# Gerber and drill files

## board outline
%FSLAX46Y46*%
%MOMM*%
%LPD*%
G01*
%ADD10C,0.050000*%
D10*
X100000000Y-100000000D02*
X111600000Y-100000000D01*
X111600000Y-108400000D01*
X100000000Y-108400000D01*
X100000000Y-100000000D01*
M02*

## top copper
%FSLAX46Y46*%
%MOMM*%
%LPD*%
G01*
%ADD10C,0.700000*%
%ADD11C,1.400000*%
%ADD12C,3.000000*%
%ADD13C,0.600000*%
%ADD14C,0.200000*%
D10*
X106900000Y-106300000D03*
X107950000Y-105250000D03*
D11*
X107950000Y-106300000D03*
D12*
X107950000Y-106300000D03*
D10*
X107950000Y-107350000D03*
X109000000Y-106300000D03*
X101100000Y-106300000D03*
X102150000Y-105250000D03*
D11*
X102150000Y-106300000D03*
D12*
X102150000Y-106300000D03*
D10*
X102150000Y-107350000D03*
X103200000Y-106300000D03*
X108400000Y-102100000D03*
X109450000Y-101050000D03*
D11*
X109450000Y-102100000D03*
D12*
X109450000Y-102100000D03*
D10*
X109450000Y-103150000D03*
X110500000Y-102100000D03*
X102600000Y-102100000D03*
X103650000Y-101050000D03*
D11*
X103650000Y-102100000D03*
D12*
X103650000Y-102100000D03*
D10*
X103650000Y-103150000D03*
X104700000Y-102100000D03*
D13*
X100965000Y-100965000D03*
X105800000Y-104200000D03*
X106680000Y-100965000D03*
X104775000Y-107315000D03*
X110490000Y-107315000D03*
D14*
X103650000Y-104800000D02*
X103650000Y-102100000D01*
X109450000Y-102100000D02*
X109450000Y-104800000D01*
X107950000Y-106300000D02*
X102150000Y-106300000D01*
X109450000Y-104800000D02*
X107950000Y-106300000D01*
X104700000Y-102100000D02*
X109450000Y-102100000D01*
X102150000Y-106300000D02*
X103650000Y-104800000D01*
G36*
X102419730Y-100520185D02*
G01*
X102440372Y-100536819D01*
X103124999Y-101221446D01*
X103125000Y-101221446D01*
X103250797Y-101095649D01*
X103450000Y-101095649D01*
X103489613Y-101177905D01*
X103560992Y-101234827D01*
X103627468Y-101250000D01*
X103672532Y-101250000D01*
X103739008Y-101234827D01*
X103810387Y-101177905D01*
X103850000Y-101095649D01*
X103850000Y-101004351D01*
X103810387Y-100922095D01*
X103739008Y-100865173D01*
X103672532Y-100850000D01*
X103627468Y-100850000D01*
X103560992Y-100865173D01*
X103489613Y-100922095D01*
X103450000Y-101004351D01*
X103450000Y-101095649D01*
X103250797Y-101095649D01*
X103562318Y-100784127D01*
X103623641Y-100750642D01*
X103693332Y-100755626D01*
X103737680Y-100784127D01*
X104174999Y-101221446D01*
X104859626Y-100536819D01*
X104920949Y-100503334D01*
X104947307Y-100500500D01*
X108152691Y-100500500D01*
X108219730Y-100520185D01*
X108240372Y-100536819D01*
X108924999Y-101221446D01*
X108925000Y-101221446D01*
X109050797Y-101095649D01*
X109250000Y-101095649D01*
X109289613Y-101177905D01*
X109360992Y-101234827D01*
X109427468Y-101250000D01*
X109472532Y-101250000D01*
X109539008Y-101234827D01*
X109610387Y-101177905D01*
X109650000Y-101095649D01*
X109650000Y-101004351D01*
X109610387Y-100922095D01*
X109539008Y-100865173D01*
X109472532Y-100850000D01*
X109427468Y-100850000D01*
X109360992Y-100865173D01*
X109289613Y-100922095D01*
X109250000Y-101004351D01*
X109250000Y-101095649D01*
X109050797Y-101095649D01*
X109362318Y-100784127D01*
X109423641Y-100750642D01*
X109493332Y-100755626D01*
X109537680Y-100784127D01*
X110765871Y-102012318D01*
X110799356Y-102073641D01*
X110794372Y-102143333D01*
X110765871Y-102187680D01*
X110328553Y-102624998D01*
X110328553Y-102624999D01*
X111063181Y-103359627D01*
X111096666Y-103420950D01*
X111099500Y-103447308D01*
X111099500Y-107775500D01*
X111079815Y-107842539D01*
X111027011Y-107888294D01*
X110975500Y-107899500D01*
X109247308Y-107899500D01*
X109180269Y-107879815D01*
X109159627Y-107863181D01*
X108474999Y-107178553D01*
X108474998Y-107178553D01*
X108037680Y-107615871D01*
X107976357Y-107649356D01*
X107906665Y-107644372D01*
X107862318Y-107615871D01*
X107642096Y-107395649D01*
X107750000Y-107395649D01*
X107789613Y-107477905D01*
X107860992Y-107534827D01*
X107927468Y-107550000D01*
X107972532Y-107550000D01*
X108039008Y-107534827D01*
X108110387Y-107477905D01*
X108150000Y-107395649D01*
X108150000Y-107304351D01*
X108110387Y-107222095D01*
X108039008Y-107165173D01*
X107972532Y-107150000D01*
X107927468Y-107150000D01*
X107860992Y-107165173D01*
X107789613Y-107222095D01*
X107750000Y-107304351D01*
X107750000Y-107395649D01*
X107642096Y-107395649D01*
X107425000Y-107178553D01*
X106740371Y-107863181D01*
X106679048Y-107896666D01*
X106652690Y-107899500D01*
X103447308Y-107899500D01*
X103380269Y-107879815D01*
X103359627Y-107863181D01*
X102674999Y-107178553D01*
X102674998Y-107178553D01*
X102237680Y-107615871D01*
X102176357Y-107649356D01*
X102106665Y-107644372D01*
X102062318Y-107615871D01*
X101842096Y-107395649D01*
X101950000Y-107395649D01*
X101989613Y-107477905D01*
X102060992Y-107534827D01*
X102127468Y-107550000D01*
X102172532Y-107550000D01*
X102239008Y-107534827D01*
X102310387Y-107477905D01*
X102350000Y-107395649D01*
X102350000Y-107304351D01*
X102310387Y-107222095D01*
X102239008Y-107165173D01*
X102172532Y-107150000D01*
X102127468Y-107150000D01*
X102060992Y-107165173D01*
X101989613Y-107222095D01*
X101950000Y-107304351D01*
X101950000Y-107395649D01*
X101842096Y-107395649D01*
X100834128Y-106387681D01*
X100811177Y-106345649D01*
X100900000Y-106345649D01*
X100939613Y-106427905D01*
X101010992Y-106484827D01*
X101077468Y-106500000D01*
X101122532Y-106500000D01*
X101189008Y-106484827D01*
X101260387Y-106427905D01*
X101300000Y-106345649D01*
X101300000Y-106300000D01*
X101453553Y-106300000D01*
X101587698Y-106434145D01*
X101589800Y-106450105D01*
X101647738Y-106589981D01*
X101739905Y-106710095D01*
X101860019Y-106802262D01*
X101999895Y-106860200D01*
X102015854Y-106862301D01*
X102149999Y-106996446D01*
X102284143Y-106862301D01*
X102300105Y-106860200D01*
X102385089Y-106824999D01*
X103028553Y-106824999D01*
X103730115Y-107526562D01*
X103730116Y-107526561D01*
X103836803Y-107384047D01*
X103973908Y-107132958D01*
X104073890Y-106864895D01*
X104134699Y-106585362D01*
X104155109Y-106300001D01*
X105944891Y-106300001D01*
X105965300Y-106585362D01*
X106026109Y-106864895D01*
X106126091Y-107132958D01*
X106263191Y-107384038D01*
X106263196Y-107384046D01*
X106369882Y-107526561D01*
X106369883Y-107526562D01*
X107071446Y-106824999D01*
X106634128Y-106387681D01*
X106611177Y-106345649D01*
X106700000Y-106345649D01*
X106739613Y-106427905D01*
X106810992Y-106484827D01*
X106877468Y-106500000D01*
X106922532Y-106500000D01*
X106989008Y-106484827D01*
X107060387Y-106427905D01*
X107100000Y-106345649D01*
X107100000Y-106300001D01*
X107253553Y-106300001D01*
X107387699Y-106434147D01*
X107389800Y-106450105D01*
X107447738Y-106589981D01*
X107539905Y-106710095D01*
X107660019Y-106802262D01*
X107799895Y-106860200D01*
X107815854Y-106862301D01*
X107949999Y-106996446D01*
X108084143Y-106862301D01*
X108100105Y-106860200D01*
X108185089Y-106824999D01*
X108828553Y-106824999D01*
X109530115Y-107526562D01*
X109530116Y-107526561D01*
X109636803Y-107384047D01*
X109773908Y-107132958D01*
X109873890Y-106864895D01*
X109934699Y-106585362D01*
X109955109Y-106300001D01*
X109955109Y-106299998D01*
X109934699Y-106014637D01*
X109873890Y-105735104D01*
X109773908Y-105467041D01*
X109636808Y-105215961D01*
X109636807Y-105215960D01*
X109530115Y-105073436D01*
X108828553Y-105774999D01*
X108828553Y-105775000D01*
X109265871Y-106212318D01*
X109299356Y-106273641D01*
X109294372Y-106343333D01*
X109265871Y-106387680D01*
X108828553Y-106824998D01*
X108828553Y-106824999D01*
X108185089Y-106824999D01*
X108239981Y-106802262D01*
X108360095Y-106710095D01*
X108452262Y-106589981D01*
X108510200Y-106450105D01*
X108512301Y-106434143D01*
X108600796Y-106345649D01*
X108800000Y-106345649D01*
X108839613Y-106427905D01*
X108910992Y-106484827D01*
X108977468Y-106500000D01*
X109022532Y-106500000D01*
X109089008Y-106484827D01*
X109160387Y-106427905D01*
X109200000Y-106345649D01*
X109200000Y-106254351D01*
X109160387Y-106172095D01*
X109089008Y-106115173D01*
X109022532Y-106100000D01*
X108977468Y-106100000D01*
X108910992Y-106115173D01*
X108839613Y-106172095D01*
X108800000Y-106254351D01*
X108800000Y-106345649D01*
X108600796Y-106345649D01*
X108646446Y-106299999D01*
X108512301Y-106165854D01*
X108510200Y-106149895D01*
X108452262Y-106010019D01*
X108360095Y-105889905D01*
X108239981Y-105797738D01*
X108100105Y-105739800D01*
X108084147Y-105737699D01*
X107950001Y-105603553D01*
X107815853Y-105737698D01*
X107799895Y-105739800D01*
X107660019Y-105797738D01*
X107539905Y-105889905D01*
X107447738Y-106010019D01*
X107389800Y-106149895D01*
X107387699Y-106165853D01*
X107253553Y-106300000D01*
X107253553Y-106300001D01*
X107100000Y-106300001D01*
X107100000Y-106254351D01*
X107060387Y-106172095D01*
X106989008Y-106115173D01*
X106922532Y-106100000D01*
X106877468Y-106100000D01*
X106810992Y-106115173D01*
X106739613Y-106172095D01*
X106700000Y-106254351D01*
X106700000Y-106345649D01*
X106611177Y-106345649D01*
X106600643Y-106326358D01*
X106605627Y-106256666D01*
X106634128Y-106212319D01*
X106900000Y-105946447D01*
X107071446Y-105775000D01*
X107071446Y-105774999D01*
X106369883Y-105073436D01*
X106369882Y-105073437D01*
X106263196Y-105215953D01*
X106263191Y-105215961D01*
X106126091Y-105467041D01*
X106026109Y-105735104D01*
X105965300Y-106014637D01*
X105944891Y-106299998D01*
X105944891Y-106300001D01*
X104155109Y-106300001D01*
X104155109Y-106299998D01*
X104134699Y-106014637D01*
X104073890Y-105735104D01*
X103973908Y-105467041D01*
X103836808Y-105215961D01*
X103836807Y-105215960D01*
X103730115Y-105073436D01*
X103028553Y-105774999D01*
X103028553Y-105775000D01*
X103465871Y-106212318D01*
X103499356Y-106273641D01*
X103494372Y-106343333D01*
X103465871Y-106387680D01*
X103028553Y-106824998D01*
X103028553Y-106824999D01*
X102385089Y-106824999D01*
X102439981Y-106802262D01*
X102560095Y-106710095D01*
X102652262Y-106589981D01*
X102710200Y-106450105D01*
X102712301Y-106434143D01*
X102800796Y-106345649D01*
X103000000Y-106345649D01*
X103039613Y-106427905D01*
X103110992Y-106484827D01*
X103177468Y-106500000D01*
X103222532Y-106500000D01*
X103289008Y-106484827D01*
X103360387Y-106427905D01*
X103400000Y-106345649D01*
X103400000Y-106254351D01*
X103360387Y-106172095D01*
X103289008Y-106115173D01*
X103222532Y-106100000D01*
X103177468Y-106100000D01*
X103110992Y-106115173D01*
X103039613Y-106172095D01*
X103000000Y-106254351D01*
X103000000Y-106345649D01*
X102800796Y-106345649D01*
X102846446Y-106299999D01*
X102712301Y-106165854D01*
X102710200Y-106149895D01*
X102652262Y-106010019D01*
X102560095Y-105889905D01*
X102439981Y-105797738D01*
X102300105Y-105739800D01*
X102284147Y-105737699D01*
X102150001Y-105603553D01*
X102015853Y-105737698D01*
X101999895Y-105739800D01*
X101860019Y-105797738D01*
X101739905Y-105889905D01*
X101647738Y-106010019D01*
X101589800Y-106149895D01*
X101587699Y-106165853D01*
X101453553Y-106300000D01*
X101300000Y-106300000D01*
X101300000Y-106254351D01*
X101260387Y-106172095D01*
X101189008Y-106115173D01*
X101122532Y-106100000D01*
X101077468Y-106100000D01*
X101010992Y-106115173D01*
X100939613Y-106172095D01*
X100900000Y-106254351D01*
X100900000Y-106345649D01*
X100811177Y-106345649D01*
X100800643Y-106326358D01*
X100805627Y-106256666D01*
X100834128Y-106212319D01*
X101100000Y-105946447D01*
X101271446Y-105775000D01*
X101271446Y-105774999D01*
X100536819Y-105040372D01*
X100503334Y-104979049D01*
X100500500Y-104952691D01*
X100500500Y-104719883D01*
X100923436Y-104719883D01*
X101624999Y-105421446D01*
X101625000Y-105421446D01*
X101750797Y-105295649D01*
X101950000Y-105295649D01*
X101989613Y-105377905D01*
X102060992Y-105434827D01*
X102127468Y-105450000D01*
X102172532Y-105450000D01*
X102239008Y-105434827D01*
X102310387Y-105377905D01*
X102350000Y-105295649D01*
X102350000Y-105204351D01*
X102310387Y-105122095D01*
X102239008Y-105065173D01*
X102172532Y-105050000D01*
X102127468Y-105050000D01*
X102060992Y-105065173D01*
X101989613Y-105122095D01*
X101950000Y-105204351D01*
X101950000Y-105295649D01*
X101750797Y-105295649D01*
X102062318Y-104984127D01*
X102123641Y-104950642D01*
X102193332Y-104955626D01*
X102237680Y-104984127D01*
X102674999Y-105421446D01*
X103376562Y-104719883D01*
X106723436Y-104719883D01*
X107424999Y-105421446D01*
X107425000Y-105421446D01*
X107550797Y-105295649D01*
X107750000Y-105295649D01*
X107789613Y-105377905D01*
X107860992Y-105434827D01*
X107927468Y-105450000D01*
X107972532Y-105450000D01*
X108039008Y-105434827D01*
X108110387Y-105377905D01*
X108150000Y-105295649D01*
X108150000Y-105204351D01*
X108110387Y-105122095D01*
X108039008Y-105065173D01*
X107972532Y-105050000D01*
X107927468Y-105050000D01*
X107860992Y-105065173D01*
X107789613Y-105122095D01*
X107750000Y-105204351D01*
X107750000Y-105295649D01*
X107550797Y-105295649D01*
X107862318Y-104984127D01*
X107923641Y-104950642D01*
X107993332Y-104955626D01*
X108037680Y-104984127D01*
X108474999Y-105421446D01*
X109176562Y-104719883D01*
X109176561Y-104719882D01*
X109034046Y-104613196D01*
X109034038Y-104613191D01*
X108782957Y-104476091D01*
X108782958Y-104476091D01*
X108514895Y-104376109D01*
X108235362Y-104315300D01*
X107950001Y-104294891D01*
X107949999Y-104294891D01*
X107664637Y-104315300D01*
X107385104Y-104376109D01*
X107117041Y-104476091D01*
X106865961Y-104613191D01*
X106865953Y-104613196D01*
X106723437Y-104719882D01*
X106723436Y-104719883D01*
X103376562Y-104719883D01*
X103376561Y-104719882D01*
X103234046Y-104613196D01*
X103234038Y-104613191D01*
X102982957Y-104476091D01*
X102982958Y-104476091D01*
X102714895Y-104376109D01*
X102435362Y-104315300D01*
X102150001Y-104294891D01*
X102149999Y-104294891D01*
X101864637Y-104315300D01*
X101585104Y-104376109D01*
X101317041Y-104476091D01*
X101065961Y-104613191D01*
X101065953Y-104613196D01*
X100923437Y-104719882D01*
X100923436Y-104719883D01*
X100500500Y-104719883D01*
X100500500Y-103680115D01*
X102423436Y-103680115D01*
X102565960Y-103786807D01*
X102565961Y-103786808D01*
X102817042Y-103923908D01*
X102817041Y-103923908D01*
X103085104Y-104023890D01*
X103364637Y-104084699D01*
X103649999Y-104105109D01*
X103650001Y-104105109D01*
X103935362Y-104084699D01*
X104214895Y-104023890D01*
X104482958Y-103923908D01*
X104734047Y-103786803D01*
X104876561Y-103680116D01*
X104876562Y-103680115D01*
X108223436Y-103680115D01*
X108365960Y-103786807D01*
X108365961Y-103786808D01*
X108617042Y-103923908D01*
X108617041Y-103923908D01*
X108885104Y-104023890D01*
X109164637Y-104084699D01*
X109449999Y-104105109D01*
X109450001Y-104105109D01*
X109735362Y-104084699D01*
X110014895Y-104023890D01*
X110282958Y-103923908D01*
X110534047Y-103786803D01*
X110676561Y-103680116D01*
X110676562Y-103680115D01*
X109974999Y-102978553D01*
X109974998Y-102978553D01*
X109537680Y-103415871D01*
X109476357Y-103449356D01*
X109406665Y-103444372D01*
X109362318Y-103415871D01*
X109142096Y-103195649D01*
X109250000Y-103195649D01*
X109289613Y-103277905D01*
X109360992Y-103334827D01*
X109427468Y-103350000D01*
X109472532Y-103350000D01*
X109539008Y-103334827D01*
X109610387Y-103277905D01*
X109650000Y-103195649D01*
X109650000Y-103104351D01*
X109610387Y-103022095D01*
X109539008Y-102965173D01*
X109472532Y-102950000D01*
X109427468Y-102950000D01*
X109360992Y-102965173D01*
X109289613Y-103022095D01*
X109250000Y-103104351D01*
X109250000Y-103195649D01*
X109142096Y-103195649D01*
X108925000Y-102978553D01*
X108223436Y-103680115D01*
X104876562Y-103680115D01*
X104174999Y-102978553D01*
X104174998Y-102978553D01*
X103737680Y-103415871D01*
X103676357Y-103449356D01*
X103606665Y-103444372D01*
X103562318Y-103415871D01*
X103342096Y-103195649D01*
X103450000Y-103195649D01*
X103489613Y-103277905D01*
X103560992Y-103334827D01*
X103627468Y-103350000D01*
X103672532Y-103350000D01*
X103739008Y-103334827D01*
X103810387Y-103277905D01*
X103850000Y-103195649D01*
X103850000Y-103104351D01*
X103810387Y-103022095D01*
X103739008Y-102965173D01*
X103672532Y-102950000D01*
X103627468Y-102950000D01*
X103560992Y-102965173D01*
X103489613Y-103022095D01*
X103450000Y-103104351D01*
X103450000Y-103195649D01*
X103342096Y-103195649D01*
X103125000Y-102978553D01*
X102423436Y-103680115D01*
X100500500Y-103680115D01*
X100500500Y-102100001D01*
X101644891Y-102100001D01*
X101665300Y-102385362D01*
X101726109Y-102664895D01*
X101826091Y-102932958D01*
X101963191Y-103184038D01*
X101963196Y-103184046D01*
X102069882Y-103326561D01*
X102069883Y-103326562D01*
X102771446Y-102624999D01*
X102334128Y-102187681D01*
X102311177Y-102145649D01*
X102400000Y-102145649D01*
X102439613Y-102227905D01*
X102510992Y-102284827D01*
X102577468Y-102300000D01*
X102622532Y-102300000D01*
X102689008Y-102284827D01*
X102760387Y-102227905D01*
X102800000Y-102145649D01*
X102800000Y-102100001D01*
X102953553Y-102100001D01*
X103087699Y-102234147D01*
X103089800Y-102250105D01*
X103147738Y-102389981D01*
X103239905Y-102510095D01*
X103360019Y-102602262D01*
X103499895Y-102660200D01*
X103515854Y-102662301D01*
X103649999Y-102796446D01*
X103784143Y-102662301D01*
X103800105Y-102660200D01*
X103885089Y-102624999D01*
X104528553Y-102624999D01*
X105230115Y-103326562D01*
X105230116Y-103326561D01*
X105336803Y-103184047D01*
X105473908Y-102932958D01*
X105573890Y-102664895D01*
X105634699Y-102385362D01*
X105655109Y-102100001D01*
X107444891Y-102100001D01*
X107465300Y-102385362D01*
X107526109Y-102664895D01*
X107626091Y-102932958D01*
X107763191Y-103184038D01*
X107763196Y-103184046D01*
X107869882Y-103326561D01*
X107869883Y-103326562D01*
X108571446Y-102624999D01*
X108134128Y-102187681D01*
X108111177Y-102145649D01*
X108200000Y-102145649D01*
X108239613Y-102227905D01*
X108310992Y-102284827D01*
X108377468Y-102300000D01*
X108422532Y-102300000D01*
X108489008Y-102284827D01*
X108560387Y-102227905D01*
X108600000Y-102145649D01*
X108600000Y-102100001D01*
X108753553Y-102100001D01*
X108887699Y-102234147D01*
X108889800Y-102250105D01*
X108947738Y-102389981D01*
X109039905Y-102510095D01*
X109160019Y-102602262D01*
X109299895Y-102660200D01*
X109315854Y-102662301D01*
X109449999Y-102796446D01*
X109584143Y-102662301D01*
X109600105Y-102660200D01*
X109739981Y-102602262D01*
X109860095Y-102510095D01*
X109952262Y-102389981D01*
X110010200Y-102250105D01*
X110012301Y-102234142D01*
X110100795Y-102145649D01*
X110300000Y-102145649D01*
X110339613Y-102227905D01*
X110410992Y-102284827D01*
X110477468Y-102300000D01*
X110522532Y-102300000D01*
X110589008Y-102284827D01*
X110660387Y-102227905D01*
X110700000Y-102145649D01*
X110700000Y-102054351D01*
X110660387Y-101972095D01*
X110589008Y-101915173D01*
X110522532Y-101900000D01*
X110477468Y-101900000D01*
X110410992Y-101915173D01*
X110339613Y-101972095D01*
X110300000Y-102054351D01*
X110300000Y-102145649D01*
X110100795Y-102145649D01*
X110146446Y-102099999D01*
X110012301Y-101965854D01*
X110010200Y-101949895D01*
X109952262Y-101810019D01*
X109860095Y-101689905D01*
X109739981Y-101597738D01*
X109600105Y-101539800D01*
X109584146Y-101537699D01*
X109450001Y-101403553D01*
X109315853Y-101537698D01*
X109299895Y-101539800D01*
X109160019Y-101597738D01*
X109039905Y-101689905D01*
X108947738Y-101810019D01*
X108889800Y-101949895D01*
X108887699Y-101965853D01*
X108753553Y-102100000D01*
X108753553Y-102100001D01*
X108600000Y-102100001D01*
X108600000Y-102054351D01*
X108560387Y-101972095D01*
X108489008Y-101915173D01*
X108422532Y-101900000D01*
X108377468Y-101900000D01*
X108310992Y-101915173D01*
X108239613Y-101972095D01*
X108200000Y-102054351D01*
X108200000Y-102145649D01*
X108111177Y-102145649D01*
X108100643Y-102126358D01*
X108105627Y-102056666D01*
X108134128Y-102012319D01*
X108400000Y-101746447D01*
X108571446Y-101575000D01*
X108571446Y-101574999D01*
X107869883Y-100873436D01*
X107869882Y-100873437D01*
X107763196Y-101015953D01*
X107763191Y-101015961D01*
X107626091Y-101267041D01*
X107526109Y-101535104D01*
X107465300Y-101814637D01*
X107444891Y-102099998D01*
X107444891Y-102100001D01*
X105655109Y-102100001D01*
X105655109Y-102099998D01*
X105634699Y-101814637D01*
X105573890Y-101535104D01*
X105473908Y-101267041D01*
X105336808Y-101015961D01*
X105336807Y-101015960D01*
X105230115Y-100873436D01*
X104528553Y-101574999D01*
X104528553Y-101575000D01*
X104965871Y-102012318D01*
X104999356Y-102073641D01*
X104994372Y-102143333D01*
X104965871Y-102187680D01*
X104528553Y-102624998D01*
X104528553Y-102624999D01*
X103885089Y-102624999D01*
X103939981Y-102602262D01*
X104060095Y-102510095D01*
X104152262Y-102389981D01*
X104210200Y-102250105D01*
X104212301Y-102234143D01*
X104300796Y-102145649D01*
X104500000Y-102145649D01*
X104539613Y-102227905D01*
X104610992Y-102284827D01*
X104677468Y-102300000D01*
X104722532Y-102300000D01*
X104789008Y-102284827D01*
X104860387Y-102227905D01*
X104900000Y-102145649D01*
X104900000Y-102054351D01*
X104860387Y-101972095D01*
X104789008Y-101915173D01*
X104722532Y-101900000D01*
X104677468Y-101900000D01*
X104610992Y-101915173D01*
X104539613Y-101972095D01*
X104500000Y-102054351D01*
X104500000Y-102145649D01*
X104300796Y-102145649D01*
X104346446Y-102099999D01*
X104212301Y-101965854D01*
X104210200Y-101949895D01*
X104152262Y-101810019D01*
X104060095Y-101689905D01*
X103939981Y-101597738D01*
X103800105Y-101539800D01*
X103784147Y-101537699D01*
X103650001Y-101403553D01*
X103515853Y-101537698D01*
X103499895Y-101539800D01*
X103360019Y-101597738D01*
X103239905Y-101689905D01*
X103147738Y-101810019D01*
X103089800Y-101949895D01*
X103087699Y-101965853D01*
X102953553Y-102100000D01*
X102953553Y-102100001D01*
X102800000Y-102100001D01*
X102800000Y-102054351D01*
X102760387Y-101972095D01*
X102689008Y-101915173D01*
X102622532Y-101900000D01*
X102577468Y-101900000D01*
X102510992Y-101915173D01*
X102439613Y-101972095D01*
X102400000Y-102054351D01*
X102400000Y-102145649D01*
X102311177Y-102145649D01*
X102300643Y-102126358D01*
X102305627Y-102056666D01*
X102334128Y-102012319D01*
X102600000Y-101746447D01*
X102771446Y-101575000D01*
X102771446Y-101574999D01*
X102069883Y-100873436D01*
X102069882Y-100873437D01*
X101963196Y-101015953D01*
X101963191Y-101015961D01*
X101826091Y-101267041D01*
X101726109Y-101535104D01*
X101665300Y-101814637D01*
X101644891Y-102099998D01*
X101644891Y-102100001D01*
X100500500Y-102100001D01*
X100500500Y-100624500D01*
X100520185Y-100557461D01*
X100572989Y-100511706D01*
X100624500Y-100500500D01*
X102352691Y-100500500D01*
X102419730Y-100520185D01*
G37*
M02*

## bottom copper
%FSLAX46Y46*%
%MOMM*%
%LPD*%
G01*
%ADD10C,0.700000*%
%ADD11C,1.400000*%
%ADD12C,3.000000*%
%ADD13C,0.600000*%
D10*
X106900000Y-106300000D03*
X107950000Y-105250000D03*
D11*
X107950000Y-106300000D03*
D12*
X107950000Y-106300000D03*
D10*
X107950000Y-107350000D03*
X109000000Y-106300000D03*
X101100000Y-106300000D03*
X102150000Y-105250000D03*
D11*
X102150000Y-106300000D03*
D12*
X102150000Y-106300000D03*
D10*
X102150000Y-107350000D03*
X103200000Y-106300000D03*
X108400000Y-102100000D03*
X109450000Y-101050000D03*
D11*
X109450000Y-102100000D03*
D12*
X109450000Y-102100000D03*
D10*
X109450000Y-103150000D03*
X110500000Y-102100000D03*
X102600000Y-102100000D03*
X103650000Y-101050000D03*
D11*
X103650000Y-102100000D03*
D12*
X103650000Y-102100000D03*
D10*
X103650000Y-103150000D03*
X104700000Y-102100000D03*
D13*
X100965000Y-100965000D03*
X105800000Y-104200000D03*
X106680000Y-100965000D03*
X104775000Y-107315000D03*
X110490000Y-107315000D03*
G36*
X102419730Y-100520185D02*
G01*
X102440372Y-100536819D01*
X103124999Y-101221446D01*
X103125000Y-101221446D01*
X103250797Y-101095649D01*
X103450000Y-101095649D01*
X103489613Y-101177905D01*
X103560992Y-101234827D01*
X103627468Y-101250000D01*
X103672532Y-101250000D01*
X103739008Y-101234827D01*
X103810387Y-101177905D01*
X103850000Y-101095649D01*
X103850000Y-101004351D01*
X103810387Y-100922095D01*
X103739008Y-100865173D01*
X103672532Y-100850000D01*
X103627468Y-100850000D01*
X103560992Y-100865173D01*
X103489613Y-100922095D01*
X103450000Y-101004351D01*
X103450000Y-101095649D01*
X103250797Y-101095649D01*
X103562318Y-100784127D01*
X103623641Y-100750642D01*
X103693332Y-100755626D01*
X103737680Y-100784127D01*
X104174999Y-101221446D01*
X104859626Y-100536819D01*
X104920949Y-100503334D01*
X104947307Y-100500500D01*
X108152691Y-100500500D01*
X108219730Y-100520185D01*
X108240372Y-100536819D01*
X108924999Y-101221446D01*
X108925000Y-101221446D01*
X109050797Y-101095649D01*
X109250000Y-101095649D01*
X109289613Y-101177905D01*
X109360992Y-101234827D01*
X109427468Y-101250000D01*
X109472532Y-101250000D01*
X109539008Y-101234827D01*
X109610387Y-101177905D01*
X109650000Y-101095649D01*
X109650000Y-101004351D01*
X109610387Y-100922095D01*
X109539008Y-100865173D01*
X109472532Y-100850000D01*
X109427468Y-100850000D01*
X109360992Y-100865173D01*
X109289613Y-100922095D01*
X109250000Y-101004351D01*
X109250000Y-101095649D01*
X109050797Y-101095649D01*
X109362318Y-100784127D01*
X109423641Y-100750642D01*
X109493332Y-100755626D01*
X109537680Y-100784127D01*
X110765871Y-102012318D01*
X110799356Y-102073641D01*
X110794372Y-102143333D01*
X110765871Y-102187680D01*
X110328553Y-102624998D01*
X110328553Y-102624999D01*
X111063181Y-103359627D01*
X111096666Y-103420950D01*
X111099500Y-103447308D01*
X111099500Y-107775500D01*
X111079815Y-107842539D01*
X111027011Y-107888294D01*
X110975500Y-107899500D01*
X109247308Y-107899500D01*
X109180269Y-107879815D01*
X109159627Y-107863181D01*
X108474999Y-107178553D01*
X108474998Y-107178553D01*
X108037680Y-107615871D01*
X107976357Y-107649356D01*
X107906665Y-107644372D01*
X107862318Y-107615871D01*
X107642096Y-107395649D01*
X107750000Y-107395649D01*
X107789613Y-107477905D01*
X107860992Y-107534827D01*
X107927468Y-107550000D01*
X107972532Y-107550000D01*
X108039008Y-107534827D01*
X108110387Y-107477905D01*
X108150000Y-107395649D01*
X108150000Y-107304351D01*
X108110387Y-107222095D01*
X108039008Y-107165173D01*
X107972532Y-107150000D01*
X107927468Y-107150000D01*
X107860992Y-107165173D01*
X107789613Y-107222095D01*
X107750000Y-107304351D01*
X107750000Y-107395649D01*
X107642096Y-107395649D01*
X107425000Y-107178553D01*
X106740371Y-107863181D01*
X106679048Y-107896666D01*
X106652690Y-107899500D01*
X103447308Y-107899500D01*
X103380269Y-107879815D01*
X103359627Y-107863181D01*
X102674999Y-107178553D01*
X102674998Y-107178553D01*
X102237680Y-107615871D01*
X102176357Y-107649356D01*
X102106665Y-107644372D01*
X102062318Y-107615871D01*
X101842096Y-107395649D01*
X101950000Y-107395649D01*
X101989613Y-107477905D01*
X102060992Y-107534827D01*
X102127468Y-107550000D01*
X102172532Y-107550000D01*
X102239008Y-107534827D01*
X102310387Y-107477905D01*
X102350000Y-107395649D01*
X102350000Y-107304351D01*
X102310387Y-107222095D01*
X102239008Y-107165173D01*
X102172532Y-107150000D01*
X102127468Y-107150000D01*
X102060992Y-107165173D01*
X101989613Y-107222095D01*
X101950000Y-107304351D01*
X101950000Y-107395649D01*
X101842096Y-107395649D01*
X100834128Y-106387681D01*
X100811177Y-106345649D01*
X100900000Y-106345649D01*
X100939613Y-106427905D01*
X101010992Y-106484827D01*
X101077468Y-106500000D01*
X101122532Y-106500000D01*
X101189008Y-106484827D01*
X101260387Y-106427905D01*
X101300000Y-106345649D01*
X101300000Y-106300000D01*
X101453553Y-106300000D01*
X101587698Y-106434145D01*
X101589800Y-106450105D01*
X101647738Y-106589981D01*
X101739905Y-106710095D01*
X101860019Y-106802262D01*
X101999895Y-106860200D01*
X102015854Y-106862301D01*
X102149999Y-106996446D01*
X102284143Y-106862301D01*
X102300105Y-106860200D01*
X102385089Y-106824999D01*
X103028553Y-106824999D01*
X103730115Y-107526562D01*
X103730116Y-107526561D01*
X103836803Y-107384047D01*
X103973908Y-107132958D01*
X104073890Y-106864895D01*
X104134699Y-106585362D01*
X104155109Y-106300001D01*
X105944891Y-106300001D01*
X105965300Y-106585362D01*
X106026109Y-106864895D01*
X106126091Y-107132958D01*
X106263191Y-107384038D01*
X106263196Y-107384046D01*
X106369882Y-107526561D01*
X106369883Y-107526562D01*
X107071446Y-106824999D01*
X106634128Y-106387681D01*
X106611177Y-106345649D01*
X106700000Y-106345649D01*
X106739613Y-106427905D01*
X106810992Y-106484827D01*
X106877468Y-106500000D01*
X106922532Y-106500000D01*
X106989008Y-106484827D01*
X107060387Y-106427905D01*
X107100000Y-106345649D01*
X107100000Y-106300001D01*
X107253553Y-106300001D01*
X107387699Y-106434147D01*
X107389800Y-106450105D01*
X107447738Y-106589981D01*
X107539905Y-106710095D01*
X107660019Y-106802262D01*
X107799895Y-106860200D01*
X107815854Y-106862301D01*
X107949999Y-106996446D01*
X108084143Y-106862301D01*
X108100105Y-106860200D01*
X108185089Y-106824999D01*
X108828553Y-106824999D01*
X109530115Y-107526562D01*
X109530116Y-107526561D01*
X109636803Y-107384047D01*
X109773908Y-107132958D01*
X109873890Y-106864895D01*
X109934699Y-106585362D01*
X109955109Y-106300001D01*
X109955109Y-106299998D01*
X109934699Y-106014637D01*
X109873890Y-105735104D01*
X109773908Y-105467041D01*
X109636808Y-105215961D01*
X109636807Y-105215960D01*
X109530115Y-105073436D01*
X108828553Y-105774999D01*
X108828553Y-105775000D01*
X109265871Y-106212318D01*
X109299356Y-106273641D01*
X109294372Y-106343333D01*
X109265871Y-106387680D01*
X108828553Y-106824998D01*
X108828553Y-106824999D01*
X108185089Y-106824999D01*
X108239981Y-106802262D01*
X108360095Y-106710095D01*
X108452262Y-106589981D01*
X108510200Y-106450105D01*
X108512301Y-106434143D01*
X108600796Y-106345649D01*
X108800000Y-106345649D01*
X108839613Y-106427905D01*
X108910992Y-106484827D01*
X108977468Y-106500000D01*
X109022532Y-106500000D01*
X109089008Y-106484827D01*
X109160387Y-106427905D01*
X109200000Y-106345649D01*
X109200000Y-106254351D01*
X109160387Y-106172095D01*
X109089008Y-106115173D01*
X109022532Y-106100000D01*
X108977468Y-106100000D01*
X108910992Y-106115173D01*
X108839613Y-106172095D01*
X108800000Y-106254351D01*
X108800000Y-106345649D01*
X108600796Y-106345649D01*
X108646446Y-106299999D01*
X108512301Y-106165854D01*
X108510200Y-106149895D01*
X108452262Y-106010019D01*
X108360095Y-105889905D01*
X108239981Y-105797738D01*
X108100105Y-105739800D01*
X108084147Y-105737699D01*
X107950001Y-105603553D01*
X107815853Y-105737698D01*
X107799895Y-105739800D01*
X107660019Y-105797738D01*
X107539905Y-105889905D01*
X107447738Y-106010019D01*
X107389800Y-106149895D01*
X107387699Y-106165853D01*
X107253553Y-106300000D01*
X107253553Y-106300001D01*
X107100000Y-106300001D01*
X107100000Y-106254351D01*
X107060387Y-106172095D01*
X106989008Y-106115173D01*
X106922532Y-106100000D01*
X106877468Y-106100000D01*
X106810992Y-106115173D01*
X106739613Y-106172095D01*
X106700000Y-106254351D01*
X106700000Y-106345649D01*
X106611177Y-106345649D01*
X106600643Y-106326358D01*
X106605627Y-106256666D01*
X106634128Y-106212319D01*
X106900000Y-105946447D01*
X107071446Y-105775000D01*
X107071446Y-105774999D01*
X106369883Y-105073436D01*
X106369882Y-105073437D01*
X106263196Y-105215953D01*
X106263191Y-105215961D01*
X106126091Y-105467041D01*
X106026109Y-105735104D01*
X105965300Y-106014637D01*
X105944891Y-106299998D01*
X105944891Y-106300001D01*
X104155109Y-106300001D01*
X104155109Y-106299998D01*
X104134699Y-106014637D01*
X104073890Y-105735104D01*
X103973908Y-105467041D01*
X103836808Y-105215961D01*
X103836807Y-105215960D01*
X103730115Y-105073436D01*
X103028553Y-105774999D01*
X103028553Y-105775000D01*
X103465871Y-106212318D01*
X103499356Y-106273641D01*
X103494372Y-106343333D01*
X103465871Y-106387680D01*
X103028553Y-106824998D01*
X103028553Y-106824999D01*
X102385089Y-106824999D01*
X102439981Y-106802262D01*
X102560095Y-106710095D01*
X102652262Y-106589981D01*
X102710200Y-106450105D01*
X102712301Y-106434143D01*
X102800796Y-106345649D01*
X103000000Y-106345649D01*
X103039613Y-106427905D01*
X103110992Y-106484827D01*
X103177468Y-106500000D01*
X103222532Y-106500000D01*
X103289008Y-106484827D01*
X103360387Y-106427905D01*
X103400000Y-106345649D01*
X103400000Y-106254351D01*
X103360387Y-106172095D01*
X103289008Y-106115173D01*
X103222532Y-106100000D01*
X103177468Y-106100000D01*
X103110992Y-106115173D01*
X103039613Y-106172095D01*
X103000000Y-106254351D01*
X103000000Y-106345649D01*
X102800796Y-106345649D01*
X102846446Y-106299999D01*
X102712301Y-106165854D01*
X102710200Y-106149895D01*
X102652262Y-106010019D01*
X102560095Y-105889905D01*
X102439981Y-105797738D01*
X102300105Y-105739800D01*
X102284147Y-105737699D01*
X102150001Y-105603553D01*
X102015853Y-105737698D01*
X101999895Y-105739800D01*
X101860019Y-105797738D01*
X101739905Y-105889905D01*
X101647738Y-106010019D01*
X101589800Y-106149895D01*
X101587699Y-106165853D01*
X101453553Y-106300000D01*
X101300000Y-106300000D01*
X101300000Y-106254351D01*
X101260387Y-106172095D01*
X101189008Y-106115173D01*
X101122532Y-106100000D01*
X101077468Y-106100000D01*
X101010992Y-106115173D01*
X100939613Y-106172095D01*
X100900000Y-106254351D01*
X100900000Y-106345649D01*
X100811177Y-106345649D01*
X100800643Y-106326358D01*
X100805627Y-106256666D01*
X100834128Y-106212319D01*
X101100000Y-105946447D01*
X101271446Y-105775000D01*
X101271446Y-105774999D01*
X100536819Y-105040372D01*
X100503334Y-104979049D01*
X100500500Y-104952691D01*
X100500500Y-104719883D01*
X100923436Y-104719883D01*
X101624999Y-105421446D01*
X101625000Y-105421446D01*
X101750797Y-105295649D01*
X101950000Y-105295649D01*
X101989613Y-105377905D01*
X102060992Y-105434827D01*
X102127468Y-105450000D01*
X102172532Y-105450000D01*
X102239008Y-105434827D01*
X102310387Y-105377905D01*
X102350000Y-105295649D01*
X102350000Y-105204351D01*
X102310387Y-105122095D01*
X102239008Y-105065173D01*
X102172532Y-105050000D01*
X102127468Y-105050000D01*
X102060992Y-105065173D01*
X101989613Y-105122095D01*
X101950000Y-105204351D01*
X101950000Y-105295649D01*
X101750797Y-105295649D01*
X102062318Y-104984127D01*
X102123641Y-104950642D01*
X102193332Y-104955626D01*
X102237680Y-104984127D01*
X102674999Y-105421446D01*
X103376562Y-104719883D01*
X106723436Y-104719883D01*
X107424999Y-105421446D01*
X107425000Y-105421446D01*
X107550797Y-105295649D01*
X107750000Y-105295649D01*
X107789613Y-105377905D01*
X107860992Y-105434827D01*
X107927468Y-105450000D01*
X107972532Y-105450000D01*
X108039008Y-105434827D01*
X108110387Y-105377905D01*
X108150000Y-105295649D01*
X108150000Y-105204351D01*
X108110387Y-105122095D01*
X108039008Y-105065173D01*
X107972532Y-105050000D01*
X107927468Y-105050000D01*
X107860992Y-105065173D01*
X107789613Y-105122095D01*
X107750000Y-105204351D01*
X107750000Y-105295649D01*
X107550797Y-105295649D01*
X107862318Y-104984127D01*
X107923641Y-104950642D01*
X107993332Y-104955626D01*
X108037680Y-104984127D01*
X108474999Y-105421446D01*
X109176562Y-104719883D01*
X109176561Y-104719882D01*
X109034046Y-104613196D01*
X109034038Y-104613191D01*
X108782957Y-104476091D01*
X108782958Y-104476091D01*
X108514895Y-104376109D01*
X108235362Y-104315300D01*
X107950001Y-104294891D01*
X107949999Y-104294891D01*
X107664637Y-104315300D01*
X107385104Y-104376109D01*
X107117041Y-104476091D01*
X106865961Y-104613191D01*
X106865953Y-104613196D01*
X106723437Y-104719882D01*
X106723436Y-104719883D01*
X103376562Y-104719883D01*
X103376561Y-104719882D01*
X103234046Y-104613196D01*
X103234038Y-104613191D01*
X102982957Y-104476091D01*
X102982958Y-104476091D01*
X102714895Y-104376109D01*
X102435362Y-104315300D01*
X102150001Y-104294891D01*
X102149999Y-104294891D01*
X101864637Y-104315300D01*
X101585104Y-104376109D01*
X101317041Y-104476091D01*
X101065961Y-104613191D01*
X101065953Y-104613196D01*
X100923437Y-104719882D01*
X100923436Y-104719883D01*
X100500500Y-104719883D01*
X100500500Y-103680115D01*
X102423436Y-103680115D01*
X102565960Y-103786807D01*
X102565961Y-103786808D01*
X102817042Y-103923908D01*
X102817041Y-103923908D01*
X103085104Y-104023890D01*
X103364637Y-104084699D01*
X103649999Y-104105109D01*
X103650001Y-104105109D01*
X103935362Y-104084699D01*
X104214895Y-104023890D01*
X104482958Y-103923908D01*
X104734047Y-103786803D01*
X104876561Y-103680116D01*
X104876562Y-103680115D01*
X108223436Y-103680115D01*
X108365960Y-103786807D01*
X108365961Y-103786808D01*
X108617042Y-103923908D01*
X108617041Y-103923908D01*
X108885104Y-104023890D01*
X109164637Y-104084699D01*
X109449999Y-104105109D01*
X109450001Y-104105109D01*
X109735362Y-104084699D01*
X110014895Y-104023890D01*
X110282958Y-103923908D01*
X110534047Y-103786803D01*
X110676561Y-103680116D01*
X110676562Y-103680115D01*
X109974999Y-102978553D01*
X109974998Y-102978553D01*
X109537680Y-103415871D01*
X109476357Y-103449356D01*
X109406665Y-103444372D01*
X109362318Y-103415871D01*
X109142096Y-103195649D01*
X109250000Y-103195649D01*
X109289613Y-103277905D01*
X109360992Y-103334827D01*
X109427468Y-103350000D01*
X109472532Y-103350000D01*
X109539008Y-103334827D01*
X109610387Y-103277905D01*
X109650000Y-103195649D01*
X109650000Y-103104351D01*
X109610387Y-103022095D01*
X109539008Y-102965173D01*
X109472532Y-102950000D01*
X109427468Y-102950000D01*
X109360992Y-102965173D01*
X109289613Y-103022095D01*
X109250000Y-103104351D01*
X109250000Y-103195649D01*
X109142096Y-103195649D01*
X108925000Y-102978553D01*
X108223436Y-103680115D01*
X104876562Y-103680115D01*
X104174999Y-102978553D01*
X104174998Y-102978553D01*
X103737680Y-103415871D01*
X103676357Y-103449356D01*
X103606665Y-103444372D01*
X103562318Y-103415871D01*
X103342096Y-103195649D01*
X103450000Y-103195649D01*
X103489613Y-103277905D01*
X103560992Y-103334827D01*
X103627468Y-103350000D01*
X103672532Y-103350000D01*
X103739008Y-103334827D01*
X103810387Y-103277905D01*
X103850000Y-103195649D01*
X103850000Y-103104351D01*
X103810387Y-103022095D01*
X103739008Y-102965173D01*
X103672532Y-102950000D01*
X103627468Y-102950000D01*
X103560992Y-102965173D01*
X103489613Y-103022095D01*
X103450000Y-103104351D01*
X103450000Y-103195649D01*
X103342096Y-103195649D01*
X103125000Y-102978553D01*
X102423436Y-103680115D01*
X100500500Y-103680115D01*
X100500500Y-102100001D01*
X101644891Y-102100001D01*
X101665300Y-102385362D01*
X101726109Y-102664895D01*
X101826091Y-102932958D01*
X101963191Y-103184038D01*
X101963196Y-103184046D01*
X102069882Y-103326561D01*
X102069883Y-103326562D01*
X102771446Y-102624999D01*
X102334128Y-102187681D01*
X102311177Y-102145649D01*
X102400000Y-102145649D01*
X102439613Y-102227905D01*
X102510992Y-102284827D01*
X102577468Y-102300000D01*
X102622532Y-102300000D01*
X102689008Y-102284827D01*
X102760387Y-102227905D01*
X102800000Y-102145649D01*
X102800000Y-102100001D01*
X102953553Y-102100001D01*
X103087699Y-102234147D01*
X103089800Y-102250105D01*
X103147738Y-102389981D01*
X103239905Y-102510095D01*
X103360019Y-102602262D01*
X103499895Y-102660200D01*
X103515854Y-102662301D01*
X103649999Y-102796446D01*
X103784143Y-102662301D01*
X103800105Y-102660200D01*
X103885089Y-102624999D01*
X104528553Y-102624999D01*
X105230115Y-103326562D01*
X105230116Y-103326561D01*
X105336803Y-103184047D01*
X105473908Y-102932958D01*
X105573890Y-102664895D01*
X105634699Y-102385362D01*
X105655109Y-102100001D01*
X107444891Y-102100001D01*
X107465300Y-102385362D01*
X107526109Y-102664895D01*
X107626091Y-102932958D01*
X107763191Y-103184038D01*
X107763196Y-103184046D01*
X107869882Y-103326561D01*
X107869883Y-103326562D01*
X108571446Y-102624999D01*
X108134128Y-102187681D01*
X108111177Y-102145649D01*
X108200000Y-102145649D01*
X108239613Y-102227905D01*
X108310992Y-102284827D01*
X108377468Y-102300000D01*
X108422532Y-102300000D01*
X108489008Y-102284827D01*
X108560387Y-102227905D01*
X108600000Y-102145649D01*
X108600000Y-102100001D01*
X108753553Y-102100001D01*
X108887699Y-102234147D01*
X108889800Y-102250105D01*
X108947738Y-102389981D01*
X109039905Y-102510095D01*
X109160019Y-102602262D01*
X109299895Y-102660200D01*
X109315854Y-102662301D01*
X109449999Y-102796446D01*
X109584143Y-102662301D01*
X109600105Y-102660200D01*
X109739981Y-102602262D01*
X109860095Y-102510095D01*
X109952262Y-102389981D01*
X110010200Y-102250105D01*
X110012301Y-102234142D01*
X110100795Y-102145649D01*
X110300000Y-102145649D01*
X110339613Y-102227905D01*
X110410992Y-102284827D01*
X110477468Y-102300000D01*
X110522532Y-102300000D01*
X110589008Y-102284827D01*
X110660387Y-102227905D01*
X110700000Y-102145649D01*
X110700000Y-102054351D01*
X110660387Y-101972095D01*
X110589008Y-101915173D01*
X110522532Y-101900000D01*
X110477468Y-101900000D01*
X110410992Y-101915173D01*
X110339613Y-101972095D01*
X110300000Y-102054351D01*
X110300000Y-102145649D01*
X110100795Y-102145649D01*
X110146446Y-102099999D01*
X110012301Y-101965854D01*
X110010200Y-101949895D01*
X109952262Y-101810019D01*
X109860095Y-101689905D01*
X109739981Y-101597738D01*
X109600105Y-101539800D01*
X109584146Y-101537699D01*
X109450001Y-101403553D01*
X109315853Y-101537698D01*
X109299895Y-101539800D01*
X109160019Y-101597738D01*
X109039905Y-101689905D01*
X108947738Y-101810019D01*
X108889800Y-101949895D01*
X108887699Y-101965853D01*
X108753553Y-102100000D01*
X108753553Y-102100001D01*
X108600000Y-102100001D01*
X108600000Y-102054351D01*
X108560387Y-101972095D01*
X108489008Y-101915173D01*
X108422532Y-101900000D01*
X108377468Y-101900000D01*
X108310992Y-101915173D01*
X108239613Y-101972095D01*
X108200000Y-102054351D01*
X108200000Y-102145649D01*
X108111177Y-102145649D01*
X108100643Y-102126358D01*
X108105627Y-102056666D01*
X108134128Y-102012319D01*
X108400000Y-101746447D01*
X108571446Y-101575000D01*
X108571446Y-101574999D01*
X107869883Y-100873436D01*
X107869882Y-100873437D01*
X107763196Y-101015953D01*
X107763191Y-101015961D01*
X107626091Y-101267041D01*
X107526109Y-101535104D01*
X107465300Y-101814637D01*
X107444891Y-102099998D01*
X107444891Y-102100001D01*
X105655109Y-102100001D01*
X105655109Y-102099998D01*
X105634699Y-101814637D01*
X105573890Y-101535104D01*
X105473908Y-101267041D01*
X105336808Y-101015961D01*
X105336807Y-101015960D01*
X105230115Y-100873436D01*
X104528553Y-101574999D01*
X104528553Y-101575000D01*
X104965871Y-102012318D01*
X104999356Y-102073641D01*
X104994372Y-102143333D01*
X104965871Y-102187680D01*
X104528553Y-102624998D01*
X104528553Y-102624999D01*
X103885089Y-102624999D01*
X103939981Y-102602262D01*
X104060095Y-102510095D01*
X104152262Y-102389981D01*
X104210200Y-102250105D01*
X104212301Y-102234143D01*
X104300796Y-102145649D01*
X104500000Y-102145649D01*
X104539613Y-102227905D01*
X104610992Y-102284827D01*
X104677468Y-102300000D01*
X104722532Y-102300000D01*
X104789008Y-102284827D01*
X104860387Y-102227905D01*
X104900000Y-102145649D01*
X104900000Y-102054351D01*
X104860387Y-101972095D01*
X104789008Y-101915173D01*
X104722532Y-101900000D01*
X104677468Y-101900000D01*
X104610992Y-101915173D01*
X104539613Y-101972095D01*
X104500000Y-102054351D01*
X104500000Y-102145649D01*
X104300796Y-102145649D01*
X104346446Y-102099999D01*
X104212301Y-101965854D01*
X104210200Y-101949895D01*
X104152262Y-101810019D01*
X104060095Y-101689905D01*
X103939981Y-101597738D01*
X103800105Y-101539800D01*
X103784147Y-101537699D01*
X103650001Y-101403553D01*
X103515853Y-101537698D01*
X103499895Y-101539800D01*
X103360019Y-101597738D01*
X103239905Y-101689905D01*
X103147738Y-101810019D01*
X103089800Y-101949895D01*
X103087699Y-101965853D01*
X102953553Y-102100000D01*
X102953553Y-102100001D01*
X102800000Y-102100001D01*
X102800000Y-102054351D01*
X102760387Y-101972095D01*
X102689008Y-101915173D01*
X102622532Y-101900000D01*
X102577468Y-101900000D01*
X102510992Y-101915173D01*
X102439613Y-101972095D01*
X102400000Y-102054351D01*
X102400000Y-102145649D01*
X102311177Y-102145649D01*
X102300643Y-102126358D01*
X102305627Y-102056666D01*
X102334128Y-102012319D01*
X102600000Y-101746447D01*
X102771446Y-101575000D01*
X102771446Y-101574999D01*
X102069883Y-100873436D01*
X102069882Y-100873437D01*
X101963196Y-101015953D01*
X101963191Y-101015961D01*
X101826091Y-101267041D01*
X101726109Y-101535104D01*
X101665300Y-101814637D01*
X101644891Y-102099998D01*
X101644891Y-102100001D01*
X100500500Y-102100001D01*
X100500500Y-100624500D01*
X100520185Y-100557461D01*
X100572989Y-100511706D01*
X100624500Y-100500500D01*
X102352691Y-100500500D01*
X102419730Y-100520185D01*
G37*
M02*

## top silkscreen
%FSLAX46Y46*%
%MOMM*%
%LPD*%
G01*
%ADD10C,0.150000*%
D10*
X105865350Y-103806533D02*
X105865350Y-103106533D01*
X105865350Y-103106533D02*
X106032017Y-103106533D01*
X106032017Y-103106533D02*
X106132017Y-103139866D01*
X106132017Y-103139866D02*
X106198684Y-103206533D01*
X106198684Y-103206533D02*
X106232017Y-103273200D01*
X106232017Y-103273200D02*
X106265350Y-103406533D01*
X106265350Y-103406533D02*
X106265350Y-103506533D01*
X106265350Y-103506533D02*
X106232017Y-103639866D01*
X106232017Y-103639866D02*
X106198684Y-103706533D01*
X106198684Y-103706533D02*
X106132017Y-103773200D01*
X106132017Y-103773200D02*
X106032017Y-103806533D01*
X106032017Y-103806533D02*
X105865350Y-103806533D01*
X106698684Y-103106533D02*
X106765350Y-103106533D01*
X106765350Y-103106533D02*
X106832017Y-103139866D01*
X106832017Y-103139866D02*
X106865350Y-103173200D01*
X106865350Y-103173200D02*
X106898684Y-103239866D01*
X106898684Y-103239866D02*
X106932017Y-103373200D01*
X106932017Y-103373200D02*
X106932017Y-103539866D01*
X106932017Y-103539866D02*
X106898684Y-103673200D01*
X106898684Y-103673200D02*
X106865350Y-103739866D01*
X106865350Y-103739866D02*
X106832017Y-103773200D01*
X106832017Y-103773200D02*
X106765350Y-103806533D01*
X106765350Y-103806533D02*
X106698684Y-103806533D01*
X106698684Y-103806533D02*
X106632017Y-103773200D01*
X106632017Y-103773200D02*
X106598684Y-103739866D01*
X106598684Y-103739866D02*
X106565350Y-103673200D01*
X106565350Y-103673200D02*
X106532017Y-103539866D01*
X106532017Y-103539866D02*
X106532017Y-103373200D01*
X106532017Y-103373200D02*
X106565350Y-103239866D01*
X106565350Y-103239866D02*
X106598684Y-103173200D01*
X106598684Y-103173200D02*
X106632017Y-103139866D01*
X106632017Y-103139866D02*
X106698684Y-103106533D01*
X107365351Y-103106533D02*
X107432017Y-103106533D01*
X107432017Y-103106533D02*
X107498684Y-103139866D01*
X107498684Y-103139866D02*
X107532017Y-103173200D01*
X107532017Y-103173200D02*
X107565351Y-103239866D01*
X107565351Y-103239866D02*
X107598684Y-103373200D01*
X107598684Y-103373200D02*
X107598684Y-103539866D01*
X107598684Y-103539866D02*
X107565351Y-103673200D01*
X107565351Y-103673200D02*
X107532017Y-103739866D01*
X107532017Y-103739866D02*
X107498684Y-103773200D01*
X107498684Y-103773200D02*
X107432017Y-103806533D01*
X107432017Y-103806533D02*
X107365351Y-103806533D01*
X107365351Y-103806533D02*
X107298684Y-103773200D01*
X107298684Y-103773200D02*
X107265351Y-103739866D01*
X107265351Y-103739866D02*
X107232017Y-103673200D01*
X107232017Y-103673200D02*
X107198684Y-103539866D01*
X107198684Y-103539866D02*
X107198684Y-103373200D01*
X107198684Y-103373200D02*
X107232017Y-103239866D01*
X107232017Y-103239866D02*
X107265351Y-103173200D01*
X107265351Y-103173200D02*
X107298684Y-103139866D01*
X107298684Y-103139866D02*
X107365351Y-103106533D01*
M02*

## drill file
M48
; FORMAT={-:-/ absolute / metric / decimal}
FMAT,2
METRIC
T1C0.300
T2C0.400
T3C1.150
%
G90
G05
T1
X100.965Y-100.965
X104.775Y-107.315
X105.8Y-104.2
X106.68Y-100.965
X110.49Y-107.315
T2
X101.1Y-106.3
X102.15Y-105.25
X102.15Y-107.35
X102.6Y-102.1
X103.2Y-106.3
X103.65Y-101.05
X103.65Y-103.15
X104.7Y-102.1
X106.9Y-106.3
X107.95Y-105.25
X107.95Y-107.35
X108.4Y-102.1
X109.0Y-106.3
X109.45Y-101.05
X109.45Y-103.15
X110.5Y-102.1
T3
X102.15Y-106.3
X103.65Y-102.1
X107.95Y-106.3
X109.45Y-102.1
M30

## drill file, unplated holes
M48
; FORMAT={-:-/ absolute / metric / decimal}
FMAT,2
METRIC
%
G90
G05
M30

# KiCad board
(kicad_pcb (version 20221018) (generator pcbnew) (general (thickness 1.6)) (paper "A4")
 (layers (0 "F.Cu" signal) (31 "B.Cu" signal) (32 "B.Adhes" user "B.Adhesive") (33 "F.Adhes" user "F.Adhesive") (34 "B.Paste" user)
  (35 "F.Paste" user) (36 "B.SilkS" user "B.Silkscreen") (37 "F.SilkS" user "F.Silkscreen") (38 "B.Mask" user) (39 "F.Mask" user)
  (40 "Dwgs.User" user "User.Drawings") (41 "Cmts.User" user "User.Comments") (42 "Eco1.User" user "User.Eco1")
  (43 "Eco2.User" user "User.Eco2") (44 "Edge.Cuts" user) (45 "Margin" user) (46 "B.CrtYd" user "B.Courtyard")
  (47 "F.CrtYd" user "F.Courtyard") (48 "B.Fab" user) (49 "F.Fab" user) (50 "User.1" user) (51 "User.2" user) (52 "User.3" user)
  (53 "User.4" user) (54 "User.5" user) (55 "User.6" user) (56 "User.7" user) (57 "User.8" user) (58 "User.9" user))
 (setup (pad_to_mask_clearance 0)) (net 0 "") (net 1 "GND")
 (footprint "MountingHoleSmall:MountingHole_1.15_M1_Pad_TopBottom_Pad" (layer "F.Cu") (at 107.95 106.3)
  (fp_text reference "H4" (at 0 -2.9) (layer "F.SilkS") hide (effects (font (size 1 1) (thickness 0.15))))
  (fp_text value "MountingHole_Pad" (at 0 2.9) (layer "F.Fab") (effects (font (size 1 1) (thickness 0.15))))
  (pad "1" thru_hole circle (at -1.05 0) (size 0.7 0.7) (drill 0.4) (layers "*.Cu" "*.Mask") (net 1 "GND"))
  (pad "1" thru_hole circle (at 0 -1.05) (size 0.7 0.7) (drill 0.4) (layers "*.Cu" "*.Mask") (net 1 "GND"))
  (pad "1" thru_hole circle (at 0 0) (size 1.4 1.4) (drill 1.15) (layers "*.Cu" "*.Mask") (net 1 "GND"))
  (pad "1" connect circle (at 0 0) (size 3 3) (layers "F.Cu" "F.Mask") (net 1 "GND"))
  (pad "1" connect circle (at 0 0) (size 3 3) (layers "B.Cu" "B.Mask") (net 1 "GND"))
  (pad "1" thru_hole circle (at 0 1.05) (size 0.7 0.7) (drill 0.4) (layers "*.Cu" "*.Mask") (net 1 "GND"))
  (pad "1" thru_hole circle (at 1.05 0) (size 0.7 0.7) (drill 0.4) (layers "*.Cu" "*.Mask") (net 1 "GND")))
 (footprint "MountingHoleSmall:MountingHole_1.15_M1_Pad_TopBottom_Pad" (layer "F.Cu") (at 102.15 106.3)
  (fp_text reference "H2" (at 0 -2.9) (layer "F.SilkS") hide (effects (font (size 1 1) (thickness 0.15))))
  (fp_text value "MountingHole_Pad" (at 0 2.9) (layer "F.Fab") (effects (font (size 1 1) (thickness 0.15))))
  (pad "1" thru_hole circle (at -1.05 0) (size 0.7 0.7) (drill 0.4) (layers "*.Cu" "*.Mask") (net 1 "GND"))
  (pad "1" thru_hole circle (at 0 -1.05) (size 0.7 0.7) (drill 0.4) (layers "*.Cu" "*.Mask") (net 1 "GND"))
  (pad "1" thru_hole circle (at 0 0) (size 1.4 1.4) (drill 1.15) (layers "*.Cu" "*.Mask") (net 1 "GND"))
  (pad "1" connect circle (at 0 0) (size 3 3) (layers "F.Cu" "F.Mask") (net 1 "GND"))
  (pad "1" connect circle (at 0 0) (size 3 3) (layers "B.Cu" "B.Mask") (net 1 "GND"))
  (pad "1" thru_hole circle (at 0 1.05) (size 0.7 0.7) (drill 0.4) (layers "*.Cu" "*.Mask") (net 1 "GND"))
  (pad "1" thru_hole circle (at 1.05 0) (size 0.7 0.7) (drill 0.4) (layers "*.Cu" "*.Mask") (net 1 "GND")))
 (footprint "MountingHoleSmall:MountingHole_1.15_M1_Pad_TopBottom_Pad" (layer "F.Cu") (at 109.45 102.1)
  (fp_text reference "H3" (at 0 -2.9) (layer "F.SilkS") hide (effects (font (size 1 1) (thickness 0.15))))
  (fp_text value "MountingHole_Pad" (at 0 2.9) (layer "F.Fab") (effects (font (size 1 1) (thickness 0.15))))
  (pad "1" thru_hole circle (at -1.05 0) (size 0.7 0.7) (drill 0.4) (layers "*.Cu" "*.Mask") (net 1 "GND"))
  (pad "1" thru_hole circle (at 0 -1.05) (size 0.7 0.7) (drill 0.4) (layers "*.Cu" "*.Mask") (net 1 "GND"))
  (pad "1" thru_hole circle (at 0 0) (size 1.4 1.4) (drill 1.15) (layers "*.Cu" "*.Mask") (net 1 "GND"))
  (pad "1" connect circle (at 0 0) (size 3 3) (layers "F.Cu" "F.Mask") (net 1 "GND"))
  (pad "1" connect circle (at 0 0) (size 3 3) (layers "B.Cu" "B.Mask") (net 1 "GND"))
  (pad "1" thru_hole circle (at 0 1.05) (size 0.7 0.7) (drill 0.4) (layers "*.Cu" "*.Mask") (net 1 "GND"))
  (pad "1" thru_hole circle (at 1.05 0) (size 0.7 0.7) (drill 0.4) (layers "*.Cu" "*.Mask") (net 1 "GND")))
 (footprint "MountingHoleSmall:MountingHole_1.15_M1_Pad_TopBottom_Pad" (layer "F.Cu") (at 103.65 102.1)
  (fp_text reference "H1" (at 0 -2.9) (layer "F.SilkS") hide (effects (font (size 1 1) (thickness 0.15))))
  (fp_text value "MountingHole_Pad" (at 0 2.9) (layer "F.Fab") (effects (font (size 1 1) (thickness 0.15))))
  (pad "1" thru_hole circle (at -1.05 0) (size 0.7 0.7) (drill 0.4) (layers "*.Cu" "*.Mask") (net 1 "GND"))
  (pad "1" thru_hole circle (at 0 -1.05) (size 0.7 0.7) (drill 0.4) (layers "*.Cu" "*.Mask") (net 1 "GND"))
  (pad "1" thru_hole circle (at 0 0) (size 1.4 1.4) (drill 1.15) (layers "*.Cu" "*.Mask") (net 1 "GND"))
  (pad "1" connect circle (at 0 0) (size 3 3) (layers "F.Cu" "F.Mask") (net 1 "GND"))
  (pad "1" connect circle (at 0 0) (size 3 3) (layers "B.Cu" "B.Mask") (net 1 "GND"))
  (pad "1" thru_hole circle (at 0 1.05) (size 0.7 0.7) (drill 0.4) (layers "*.Cu" "*.Mask") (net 1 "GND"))
  (pad "1" thru_hole circle (at 1.05 0) (size 0.7 0.7) (drill 0.4) (layers "*.Cu" "*.Mask") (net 1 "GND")))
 (gr_rect (start 100 100) (end 111.6 108.4) (stroke (width 0.05) (type default)) (fill none) (layer "Edge.Cuts"))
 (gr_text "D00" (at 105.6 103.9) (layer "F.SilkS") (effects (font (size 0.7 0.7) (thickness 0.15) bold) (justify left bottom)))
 (segment (start 103.65 104.8) (end 103.65 102.1) (width 0.2) (layer "F.Cu") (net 1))
 (segment (start 109.45 102.1) (end 109.45 104.8) (width 0.2) (layer "F.Cu") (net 1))
 (segment (start 107.95 106.3) (end 102.15 106.3) (width 0.2) (layer "F.Cu") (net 1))
 (segment (start 109.45 104.8) (end 107.95 106.3) (width 0.2) (layer "F.Cu") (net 1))
 (segment (start 104.7 102.1) (end 109.45 102.1) (width 0.2) (layer "F.Cu") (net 1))
 (segment (start 102.15 106.3) (end 103.65 104.8) (width 0.2) (layer "F.Cu") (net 1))
 (via (at 100.965 100.965) (size 0.6) (drill 0.3) (layers "F.Cu" "B.Cu") (free) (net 1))
 (via (at 105.8 104.2) (size 0.6) (drill 0.3) (layers "F.Cu" "B.Cu") (free) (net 1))
 (via (at 106.68 100.965) (size 0.6) (drill 0.3) (layers "F.Cu" "B.Cu") (free) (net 1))
 (via (at 104.775 107.315) (size 0.6) (drill 0.3) (layers "F.Cu" "B.Cu") (free) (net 1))
 (via (at 110.49 107.315) (size 0.6) (drill 0.3) (layers "F.Cu" "B.Cu") (free) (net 1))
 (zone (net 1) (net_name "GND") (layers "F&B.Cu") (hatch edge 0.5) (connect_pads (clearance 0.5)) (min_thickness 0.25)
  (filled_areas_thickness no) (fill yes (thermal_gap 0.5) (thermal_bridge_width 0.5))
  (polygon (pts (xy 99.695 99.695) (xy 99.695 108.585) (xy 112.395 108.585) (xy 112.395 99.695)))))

